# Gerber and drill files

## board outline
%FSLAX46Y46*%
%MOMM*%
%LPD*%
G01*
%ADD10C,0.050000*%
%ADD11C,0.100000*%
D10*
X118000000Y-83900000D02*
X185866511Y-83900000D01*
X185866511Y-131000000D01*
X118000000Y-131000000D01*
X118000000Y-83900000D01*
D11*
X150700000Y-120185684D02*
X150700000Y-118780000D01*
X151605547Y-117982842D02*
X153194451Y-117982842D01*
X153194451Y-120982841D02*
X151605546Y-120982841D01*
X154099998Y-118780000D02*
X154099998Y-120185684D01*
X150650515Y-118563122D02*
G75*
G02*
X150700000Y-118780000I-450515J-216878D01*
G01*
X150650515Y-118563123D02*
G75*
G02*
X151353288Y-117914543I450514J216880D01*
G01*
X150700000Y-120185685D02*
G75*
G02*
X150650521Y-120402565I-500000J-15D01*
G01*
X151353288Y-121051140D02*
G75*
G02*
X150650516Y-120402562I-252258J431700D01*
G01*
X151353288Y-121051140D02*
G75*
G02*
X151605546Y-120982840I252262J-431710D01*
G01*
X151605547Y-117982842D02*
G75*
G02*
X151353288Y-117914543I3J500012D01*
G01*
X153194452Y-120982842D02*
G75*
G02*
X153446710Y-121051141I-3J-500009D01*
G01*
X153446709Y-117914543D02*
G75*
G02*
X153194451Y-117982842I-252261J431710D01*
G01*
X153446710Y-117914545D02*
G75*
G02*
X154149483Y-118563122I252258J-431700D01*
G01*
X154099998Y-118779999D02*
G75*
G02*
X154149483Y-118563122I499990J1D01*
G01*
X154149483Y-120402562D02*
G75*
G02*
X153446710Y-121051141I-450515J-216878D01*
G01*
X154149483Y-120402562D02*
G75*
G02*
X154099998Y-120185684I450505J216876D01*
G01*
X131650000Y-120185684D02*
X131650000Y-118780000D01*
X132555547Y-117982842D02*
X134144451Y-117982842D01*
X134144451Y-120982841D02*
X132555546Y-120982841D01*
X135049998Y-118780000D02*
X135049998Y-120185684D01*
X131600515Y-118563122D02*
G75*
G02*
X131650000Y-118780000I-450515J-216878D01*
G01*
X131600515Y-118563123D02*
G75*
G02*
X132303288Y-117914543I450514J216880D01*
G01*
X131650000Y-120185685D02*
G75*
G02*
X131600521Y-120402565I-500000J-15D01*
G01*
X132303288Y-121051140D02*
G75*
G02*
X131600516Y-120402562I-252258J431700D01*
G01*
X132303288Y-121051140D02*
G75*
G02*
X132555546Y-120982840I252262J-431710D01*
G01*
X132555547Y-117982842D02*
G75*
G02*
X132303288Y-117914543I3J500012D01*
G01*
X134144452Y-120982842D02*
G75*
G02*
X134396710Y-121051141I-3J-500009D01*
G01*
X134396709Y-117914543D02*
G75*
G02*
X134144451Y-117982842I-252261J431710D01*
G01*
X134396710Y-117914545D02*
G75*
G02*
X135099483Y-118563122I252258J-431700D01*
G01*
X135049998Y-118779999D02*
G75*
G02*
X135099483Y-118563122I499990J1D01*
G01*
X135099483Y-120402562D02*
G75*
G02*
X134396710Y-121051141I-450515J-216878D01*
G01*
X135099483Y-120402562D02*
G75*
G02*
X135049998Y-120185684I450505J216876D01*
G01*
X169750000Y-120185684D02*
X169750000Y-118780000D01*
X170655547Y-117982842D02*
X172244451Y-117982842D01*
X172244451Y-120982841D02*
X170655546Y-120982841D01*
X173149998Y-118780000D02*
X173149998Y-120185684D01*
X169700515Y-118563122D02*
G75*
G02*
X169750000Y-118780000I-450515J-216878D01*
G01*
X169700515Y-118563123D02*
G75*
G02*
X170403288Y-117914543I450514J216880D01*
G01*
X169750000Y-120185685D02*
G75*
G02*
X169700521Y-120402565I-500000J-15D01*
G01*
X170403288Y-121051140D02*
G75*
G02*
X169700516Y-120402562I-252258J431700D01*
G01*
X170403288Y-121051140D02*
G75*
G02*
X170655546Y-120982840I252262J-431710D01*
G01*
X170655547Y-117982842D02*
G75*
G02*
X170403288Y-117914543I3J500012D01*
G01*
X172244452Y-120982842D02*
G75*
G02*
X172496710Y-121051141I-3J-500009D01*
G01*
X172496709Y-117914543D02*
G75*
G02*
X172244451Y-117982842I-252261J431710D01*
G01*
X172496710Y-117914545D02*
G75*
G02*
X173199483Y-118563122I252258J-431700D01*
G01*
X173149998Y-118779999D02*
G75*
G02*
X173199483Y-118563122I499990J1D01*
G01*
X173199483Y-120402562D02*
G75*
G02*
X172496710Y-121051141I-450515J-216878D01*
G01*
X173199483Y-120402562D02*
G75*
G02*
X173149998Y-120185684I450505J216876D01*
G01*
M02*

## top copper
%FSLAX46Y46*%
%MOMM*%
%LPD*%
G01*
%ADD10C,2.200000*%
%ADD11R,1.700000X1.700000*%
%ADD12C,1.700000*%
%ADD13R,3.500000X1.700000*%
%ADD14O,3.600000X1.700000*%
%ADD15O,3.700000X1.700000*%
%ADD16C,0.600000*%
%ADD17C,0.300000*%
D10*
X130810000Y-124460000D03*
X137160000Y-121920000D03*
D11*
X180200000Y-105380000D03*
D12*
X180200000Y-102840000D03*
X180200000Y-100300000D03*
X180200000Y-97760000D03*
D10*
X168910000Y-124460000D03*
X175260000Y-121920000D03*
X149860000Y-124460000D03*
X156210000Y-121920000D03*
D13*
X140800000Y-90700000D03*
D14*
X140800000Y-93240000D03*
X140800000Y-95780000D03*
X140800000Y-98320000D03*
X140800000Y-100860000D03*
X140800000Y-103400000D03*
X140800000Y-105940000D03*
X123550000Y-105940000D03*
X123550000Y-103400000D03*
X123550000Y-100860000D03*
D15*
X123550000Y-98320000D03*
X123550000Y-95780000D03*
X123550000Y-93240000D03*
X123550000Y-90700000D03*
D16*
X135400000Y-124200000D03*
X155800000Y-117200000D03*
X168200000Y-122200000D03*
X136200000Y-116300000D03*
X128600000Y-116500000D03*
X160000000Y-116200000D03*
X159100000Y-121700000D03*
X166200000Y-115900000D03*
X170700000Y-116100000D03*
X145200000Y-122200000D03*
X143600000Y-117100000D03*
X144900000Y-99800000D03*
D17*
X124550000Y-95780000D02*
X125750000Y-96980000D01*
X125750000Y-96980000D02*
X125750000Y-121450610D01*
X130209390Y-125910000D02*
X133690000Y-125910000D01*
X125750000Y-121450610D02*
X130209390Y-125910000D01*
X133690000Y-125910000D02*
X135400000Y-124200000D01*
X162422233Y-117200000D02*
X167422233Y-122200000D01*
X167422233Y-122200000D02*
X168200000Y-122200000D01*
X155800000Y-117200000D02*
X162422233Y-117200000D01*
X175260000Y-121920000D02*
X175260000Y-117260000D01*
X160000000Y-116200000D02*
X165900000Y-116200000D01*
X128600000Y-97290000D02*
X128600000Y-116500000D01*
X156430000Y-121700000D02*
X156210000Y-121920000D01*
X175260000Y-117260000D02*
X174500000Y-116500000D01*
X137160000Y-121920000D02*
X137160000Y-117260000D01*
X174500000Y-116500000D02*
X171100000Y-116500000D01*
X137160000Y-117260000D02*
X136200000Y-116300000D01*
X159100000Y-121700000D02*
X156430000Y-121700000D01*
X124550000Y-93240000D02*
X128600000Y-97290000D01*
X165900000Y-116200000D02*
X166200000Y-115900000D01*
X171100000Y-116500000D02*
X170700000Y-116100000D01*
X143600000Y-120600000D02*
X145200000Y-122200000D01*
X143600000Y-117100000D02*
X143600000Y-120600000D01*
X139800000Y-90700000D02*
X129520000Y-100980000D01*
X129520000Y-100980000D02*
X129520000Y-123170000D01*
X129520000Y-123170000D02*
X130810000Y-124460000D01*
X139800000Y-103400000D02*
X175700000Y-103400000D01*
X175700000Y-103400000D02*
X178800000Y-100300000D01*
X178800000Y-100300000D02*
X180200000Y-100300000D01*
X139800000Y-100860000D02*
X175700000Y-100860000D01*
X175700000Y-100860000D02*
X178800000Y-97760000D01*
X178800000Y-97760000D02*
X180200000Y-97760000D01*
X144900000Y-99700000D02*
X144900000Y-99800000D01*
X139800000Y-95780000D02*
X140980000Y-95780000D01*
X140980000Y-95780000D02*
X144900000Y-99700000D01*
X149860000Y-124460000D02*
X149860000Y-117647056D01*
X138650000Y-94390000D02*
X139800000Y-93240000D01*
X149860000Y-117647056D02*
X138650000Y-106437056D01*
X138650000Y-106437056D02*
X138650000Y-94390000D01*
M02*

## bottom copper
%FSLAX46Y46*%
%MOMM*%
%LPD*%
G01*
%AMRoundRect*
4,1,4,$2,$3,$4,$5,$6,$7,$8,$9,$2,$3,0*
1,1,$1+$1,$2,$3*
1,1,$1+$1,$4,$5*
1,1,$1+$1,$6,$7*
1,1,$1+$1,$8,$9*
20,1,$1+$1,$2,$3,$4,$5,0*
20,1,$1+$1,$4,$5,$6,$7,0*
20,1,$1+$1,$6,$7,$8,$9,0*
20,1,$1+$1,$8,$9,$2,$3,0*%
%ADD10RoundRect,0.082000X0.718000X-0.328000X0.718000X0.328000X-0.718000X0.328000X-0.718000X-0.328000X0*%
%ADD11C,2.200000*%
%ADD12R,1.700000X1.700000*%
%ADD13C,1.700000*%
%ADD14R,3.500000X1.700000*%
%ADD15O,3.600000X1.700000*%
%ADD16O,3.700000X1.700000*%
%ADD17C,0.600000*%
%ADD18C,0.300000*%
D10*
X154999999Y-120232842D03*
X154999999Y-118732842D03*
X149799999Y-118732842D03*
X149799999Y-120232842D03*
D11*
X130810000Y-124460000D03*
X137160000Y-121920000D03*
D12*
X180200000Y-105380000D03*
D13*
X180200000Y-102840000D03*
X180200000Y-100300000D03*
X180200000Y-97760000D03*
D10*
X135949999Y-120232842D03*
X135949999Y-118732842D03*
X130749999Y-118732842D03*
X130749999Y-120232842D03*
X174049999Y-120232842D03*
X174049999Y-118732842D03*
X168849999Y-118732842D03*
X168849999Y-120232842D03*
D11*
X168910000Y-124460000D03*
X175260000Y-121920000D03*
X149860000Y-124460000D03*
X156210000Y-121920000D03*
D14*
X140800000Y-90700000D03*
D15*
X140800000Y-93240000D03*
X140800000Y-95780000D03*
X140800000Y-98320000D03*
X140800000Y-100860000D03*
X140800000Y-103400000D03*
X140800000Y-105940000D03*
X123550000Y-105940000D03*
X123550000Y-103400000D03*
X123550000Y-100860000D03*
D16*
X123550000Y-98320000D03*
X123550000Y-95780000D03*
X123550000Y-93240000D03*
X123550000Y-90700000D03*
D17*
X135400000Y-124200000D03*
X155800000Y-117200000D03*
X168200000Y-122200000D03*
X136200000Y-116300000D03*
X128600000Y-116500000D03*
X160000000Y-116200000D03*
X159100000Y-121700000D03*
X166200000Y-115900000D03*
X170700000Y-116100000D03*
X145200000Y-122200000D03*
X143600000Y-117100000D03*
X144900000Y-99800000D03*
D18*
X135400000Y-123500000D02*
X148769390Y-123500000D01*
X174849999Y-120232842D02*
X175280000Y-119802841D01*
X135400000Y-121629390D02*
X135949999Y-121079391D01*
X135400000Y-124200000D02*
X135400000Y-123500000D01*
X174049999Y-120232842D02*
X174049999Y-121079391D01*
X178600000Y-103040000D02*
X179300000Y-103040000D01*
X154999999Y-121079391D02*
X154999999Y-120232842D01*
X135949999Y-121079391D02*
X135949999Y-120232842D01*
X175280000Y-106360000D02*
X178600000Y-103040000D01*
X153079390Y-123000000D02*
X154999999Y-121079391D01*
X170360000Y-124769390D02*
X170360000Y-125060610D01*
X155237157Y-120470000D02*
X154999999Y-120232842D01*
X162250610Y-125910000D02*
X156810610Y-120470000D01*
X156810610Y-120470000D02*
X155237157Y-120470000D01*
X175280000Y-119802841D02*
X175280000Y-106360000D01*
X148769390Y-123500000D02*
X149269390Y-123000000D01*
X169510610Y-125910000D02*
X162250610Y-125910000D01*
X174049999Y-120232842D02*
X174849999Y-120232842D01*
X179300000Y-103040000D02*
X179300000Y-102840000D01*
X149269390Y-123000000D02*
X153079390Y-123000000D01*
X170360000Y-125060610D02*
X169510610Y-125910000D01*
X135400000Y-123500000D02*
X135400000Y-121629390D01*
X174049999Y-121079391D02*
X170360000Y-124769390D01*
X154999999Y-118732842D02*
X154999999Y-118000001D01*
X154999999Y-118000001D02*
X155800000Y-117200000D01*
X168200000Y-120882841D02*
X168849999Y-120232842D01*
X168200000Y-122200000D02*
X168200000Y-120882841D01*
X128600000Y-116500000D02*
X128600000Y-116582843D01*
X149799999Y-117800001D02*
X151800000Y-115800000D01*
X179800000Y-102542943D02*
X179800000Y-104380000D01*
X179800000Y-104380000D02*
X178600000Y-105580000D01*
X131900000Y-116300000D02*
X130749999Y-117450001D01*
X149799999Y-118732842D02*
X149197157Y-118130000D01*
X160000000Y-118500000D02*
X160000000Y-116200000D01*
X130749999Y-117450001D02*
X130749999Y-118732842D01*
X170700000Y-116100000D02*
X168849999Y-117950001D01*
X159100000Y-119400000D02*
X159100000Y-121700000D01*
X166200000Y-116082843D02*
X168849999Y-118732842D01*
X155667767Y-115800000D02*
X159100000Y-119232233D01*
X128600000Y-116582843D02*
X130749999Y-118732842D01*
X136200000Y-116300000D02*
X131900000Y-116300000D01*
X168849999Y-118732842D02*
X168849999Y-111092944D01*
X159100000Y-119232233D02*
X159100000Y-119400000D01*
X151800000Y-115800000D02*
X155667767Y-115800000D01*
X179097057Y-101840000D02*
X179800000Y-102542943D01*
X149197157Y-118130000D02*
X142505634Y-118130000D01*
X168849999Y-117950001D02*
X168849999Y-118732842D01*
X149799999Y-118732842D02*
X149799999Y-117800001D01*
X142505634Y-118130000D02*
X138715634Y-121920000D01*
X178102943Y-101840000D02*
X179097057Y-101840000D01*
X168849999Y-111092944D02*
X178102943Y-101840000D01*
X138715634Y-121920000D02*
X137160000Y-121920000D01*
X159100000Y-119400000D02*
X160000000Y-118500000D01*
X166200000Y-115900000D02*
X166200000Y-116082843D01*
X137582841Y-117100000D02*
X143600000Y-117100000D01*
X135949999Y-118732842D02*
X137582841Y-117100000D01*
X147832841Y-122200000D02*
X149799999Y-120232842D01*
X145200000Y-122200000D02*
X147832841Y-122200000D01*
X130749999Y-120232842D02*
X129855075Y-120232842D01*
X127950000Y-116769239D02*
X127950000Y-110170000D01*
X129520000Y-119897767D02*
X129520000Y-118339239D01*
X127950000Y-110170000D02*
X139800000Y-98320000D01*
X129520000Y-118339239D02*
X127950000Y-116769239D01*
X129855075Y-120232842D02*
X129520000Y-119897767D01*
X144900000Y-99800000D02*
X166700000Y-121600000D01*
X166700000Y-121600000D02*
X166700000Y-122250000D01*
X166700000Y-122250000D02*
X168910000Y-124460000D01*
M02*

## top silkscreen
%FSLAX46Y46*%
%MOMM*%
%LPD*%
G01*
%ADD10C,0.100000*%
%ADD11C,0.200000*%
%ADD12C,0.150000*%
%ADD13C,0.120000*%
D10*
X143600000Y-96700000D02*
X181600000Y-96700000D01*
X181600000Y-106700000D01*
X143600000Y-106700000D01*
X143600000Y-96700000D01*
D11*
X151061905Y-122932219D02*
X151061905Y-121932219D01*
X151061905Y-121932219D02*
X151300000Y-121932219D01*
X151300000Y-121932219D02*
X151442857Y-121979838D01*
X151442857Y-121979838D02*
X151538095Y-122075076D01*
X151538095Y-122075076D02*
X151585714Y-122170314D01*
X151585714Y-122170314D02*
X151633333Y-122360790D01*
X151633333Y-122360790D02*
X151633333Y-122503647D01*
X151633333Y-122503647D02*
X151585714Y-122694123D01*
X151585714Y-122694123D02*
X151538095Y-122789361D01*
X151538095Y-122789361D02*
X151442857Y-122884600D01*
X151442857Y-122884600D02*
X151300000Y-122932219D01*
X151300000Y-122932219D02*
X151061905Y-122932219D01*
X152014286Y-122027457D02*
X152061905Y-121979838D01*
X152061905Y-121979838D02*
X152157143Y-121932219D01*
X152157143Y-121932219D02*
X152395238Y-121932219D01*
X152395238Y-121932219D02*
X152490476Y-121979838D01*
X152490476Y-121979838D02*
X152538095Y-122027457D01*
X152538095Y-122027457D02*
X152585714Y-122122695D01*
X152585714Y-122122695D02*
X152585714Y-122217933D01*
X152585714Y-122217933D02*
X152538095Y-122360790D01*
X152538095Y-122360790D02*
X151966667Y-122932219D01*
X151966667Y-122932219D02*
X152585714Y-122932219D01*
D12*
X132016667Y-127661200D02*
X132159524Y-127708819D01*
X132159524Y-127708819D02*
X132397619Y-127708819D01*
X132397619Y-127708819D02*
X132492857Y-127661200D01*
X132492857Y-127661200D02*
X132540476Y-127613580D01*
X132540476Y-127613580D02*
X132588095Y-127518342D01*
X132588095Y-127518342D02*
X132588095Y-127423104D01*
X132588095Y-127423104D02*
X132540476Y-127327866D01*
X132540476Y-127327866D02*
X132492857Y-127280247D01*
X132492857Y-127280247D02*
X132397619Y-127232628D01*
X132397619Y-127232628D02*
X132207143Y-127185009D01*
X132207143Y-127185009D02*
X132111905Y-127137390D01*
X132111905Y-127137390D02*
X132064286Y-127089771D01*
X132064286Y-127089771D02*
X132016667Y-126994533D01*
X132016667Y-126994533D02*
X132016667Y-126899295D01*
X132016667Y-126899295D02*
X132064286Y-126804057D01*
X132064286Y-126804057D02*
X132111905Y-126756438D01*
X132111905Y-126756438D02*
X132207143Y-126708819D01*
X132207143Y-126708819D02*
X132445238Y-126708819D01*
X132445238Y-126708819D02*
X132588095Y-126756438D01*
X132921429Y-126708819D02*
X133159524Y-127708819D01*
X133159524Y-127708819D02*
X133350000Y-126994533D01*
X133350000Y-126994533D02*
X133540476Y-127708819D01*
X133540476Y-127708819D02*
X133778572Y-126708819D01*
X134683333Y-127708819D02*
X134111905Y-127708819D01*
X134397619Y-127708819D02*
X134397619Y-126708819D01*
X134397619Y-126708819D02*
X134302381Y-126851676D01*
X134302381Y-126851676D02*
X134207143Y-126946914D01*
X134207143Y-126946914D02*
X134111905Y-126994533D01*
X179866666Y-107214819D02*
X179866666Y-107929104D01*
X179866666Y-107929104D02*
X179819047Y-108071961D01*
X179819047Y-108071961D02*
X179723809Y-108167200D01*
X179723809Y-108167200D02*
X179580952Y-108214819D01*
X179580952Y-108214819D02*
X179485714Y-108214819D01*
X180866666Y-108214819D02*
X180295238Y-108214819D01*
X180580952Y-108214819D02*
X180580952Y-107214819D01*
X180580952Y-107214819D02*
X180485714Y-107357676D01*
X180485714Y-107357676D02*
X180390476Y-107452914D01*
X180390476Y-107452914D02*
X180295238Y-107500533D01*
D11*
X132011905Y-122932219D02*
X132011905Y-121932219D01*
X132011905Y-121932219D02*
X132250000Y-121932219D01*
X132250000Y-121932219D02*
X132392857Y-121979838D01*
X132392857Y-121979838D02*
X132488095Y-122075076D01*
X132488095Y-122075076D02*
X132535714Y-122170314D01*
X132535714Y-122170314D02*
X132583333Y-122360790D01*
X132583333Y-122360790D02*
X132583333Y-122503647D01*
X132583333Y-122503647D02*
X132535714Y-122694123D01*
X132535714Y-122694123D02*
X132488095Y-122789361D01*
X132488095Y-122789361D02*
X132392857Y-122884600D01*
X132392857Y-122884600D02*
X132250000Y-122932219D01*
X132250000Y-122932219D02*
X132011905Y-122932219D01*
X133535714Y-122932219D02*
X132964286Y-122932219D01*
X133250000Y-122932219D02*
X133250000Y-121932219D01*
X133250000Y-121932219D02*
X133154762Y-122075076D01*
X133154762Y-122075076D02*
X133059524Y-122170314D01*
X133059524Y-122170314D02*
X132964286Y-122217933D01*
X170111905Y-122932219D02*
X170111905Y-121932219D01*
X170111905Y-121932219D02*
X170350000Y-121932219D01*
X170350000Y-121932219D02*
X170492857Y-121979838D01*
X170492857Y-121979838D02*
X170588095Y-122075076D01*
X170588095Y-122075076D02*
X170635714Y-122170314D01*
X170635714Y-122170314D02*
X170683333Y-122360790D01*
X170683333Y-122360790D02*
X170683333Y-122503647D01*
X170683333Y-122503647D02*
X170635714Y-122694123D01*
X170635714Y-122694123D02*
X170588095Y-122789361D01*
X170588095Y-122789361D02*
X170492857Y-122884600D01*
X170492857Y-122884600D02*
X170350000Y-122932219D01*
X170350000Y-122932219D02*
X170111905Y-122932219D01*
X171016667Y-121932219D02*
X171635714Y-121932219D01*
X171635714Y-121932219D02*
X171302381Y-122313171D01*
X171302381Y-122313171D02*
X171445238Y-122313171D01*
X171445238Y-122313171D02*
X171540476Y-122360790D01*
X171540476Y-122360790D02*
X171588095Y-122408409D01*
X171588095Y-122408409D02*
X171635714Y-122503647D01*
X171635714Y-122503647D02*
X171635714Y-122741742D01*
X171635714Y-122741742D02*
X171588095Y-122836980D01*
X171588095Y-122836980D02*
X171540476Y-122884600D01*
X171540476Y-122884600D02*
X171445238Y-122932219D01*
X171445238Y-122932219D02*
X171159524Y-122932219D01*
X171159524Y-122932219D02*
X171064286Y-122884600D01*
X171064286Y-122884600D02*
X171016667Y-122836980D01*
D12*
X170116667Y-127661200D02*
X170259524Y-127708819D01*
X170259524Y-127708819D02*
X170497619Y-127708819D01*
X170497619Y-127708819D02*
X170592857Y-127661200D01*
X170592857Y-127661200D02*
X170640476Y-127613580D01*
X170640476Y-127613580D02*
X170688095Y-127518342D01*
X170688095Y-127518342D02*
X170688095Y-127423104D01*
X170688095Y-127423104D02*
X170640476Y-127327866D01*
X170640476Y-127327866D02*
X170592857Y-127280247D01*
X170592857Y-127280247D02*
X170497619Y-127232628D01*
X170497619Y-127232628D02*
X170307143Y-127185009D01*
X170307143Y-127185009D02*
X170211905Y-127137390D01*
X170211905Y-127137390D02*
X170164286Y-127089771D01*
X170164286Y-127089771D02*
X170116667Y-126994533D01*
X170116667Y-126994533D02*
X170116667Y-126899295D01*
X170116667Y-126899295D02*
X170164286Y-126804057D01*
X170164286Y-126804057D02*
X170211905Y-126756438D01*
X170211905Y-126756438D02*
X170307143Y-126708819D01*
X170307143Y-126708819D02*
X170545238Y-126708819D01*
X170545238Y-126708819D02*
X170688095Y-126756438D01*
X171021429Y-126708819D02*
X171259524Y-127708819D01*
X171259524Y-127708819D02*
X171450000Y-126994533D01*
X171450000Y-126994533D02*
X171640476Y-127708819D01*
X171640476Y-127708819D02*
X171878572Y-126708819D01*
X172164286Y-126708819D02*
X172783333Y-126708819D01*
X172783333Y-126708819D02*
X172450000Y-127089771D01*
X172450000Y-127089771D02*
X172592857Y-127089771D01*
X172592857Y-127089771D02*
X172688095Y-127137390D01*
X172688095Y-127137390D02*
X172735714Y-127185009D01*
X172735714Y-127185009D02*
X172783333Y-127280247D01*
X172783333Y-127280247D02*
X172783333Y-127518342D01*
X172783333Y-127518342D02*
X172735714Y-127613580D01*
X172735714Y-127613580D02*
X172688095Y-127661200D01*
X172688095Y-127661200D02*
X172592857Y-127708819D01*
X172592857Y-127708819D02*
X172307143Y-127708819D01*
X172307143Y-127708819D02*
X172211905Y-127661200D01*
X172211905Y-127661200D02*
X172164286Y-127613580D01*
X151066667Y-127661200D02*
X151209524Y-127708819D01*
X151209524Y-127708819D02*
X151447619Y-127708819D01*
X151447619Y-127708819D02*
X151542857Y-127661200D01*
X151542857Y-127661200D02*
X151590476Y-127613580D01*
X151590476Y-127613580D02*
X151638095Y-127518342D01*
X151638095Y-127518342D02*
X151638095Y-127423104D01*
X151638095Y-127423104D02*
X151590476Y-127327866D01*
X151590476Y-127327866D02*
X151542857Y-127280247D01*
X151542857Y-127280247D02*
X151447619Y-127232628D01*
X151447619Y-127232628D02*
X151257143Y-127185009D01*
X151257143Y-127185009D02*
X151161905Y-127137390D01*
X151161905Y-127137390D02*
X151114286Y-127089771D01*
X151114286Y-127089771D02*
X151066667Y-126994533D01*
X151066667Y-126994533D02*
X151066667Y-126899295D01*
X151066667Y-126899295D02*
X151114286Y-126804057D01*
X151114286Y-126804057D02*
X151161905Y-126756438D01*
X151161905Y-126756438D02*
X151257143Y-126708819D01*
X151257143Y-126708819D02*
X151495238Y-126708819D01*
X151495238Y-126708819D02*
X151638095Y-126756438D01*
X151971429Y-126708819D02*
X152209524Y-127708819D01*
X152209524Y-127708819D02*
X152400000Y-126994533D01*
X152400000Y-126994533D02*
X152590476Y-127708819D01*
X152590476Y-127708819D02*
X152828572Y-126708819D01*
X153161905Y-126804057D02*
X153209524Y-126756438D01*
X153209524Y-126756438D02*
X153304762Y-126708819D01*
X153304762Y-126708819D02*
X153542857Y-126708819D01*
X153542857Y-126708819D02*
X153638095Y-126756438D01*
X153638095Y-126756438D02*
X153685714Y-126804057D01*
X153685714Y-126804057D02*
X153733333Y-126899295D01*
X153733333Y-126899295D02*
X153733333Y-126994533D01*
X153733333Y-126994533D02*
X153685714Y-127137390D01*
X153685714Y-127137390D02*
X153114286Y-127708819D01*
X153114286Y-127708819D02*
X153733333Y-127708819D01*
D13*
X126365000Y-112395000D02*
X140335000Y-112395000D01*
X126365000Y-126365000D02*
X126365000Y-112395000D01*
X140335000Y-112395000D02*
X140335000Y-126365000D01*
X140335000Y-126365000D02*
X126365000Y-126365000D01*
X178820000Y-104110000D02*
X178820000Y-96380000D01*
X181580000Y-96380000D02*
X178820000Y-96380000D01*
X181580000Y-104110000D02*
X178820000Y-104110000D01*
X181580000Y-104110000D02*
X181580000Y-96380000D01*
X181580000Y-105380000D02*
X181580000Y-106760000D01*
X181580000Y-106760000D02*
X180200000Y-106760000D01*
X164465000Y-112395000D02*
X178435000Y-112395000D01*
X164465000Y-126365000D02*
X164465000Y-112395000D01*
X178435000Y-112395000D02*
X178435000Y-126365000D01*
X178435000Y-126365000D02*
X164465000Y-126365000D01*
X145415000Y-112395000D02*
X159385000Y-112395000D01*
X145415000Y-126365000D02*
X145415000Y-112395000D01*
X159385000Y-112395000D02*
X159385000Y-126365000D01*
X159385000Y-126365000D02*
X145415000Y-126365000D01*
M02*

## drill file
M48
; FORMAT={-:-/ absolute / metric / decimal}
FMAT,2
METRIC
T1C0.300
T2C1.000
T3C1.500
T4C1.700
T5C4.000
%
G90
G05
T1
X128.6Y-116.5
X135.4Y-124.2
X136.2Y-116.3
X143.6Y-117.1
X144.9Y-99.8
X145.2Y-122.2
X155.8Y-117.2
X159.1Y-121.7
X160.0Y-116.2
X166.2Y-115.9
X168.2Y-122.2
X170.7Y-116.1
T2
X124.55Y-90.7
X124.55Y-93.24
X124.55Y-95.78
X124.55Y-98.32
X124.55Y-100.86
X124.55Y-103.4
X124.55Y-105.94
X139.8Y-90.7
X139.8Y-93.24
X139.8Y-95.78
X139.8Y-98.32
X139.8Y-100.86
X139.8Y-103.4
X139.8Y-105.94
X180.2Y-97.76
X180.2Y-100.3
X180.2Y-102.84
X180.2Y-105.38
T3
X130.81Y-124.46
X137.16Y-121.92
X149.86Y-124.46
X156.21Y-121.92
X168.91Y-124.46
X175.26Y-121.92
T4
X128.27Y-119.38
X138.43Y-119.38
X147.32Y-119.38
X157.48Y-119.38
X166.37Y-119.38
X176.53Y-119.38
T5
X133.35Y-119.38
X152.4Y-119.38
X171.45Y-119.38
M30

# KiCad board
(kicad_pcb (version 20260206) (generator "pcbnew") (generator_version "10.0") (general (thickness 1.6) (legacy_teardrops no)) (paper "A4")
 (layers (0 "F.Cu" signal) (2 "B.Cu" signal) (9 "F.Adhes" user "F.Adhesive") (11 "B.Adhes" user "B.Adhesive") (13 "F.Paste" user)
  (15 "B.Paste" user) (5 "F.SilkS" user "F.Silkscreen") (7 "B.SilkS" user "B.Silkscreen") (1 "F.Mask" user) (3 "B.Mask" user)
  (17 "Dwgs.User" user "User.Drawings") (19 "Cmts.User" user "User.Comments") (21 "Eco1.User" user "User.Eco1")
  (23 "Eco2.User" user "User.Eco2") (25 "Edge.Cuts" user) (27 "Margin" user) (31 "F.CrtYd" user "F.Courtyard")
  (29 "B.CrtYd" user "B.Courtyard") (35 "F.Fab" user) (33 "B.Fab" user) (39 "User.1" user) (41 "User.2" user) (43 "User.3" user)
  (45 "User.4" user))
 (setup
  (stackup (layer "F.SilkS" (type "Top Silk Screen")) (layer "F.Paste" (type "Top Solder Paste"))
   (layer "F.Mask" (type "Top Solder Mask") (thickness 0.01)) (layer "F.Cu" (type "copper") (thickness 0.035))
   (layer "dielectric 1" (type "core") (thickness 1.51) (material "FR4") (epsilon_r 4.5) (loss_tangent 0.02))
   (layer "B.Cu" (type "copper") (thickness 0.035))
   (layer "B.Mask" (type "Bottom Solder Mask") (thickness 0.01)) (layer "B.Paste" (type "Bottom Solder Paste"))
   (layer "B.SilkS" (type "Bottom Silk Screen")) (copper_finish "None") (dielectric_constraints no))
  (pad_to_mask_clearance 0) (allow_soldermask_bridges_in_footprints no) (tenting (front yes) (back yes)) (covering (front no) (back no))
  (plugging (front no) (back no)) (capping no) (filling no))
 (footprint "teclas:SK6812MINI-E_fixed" (layer "F.Cu") (at 152.4 119.38 180)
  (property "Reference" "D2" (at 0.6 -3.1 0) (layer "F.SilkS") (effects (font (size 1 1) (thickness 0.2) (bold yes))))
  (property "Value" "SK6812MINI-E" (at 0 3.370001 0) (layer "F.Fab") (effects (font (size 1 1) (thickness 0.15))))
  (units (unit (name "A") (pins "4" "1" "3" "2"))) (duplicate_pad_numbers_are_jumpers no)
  (fp_line (start 1.7 -0.805684) (end 1.7 0.6) (stroke (width 0.1) (type solid)) (layer "Edge.Cuts"))
  (fp_line (start 0.794453 1.397158) (end -0.794451 1.397158) (stroke (width 0.1) (type solid)) (layer "Edge.Cuts"))
  (fp_line (start -0.794451 -1.602841) (end 0.794454 -1.602841) (stroke (width 0.1) (type solid)) (layer "Edge.Cuts"))
  (fp_line (start -1.699998 0.6) (end -1.699998 -0.805684) (stroke (width 0.1) (type solid)) (layer "Edge.Cuts"))
  (fp_arc (start 1.749485 0.816878) (mid 1.712528 0.711226) (end 1.7 0.6) (stroke (width 0.1) (type solid)) (layer "Edge.Cuts"))
  (fp_arc (start 1.749485 0.816877) (mid 1.638073 1.401193) (end 1.046712 1.465457) (stroke (width 0.1) (type solid)) (layer "Edge.Cuts"))
  (fp_arc (start 1.7 -0.805685) (mid 1.712528 -0.91691) (end 1.749485 -1.022562) (stroke (width 0.1) (type solid)) (layer "Edge.Cuts"))
  (fp_arc (start 1.046712 -1.67114) (mid 1.638072 -1.606876) (end 1.749485 -1.022562) (stroke (width 0.1) (type solid)) (layer "Edge.Cuts"))
  (fp_arc (start 1.046712 -1.67114) (mid 0.925124 -1.620218) (end 0.794454 -1.602841) (stroke (width 0.1) (type solid)) (layer "Edge.Cuts"))
  (fp_arc (start 0.794453 1.397158) (mid 0.925124 1.414535) (end 1.046712 1.465457) (stroke (width 0.1) (type solid)) (layer "Edge.Cuts"))
  (fp_arc (start -0.794452 -1.602842) (mid -0.925122 -1.620219) (end -1.04671 -1.671141) (stroke (width 0.1) (type solid))
   (layer "Edge.Cuts"))
  (fp_arc (start -1.046709 1.465457) (mid -0.925121 1.414535) (end -0.794451 1.397158) (stroke (width 0.1) (type solid)) (layer "Edge.Cuts"))
  (fp_arc (start -1.04671 1.465455) (mid -1.638069 1.401192) (end -1.749483 0.816878) (stroke (width 0.1) (type solid)) (layer "Edge.Cuts"))
  (fp_arc (start -1.699998 0.600001) (mid -1.712526 0.711226) (end -1.749483 0.816878) (stroke (width 0.1) (type solid)) (layer "Edge.Cuts"))
  (fp_arc (start -1.749483 -1.022562) (mid -1.63807 -1.606877) (end -1.04671 -1.671141) (stroke (width 0.1) (type solid))
   (layer "Edge.Cuts"))
  (fp_arc (start -1.749483 -1.022562) (mid -1.712526 -0.91691) (end -1.699998 -0.805684) (stroke (width 0.1) (type solid))
   (layer "Edge.Cuts"))
  (pad "1" smd roundrect (at -2.599999 -0.852842 90) (size 0.82 1.6) (layers "B.Cu" "B.Mask" "B.Paste") (roundrect_rratio 0.1) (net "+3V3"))
  (pad "2" smd roundrect (at -2.599999 0.647158 90) (size 0.82 1.6) (layers "B.Cu" "B.Mask" "B.Paste") (roundrect_rratio 0.1)
   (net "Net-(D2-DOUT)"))
  (pad "3" smd roundrect (at 2.600001 0.647158 90) (size 0.82 1.6) (layers "B.Cu" "B.Mask" "B.Paste") (roundrect_rratio 0.1) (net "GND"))
  (pad "4" smd roundrect (at 2.600001 -0.852842 90) (size 0.82 1.6) (layers "B.Cu" "B.Mask" "B.Paste") (roundrect_rratio 0.1)
   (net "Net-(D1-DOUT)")))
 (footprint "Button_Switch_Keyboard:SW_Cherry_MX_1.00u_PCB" (layer "F.Cu") (at 130.81 124.46 180)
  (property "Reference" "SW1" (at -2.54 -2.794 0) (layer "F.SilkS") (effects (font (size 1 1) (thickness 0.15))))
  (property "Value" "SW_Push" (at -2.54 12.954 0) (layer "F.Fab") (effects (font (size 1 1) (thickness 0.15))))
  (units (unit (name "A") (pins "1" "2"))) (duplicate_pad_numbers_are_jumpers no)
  (fp_line (start 4.445 12.065) (end -9.525 12.065) (stroke (width 0.12) (type solid)) (layer "F.SilkS"))
  (fp_line (start 4.445 -1.905) (end 4.445 12.065) (stroke (width 0.12) (type solid)) (layer "F.SilkS"))
  (fp_line (start -9.525 12.065) (end -9.525 -1.905) (stroke (width 0.12) (type solid)) (layer "F.SilkS"))
  (fp_line (start -9.525 -1.905) (end 4.445 -1.905) (stroke (width 0.12) (type solid)) (layer "F.SilkS"))
  (pad "" np_thru_hole circle (at -7.62 5.08 180) (size 1.7 1.7) (drill 1.7) (layers "*.Cu" "*.Mask"))
  (pad "" np_thru_hole circle (at -2.54 5.08 180) (size 4 4) (drill 4) (layers "*.Cu" "*.Mask"))
  (pad "" np_thru_hole circle (at 2.54 5.08 180) (size 1.7 1.7) (drill 1.7) (layers "*.Cu" "*.Mask"))
  (pad "1" thru_hole circle (at 0 0 180) (size 2.2 2.2) (drill 1.5) (layers "*.Cu" "*.Mask") (remove_unused_layers no)
   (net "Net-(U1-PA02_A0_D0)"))
  (pad "2" thru_hole circle (at -6.35 2.54 180) (size 2.2 2.2) (drill 1.5) (layers "*.Cu" "*.Mask") (remove_unused_layers no) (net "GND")))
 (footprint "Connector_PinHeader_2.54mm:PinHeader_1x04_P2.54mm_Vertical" (layer "F.Cu") (at 180.2 105.38 180)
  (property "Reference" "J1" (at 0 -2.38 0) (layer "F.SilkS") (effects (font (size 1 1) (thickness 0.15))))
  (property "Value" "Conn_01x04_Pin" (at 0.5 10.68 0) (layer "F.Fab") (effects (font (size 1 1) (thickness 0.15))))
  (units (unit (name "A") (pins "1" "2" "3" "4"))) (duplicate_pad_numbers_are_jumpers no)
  (fp_line (start 1.38 1.27) (end 1.38 9) (stroke (width 0.12) (type solid)) (layer "F.SilkS"))
  (fp_line (start -1.38 9) (end 1.38 9) (stroke (width 0.12) (type solid)) (layer "F.SilkS"))
  (fp_line (start -1.38 1.27) (end 1.38 1.27) (stroke (width 0.12) (type solid)) (layer "F.SilkS"))
  (fp_line (start -1.38 1.27) (end -1.38 9) (stroke (width 0.12) (type solid)) (layer "F.SilkS"))
  (fp_line (start -1.38 0) (end -1.38 -1.38) (stroke (width 0.12) (type solid)) (layer "F.SilkS"))
  (fp_line (start -1.38 -1.38) (end 0 -1.38) (stroke (width 0.12) (type solid)) (layer "F.SilkS"))
  (pad "1" thru_hole rect (at 0 0 180) (size 1.7 1.7) (drill 1) (layers "*.Cu" "*.Mask") (remove_unused_layers no) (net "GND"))
  (pad "2" thru_hole circle (at 0 2.54 180) (size 1.7 1.7) (drill 1) (layers "*.Cu" "*.Mask") (remove_unused_layers no) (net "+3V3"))
  (pad "3" thru_hole circle (at 0 5.08 180) (size 1.7 1.7) (drill 1) (layers "*.Cu" "*.Mask") (remove_unused_layers no)
   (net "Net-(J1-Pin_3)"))
  (pad "4" thru_hole circle (at 0 7.62 180) (size 1.7 1.7) (drill 1) (layers "*.Cu" "*.Mask") (remove_unused_layers no)
   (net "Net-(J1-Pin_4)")))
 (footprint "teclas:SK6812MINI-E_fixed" (layer "F.Cu") (at 133.35 119.38 180)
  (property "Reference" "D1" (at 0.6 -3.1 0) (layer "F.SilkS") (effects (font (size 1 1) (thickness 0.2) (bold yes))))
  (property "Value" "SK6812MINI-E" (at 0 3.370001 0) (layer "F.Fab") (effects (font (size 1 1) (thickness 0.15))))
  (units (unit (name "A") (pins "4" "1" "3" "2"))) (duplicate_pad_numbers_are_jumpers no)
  (fp_line (start 1.7 -0.805684) (end 1.7 0.6) (stroke (width 0.1) (type solid)) (layer "Edge.Cuts"))
  (fp_line (start 0.794453 1.397158) (end -0.794451 1.397158) (stroke (width 0.1) (type solid)) (layer "Edge.Cuts"))
  (fp_line (start -0.794451 -1.602841) (end 0.794454 -1.602841) (stroke (width 0.1) (type solid)) (layer "Edge.Cuts"))
  (fp_line (start -1.699998 0.6) (end -1.699998 -0.805684) (stroke (width 0.1) (type solid)) (layer "Edge.Cuts"))
  (fp_arc (start 1.749485 0.816878) (mid 1.712528 0.711226) (end 1.7 0.6) (stroke (width 0.1) (type solid)) (layer "Edge.Cuts"))
  (fp_arc (start 1.749485 0.816877) (mid 1.638073 1.401193) (end 1.046712 1.465457) (stroke (width 0.1) (type solid)) (layer "Edge.Cuts"))
  (fp_arc (start 1.7 -0.805685) (mid 1.712528 -0.91691) (end 1.749485 -1.022562) (stroke (width 0.1) (type solid)) (layer "Edge.Cuts"))
  (fp_arc (start 1.046712 -1.67114) (mid 1.638072 -1.606876) (end 1.749485 -1.022562) (stroke (width 0.1) (type solid)) (layer "Edge.Cuts"))
  (fp_arc (start 1.046712 -1.67114) (mid 0.925124 -1.620218) (end 0.794454 -1.602841) (stroke (width 0.1) (type solid)) (layer "Edge.Cuts"))
  (fp_arc (start 0.794453 1.397158) (mid 0.925124 1.414535) (end 1.046712 1.465457) (stroke (width 0.1) (type solid)) (layer "Edge.Cuts"))
  (fp_arc (start -0.794452 -1.602842) (mid -0.925122 -1.620219) (end -1.04671 -1.671141) (stroke (width 0.1) (type solid))
   (layer "Edge.Cuts"))
  (fp_arc (start -1.046709 1.465457) (mid -0.925121 1.414535) (end -0.794451 1.397158) (stroke (width 0.1) (type solid)) (layer "Edge.Cuts"))
  (fp_arc (start -1.04671 1.465455) (mid -1.638069 1.401192) (end -1.749483 0.816878) (stroke (width 0.1) (type solid)) (layer "Edge.Cuts"))
  (fp_arc (start -1.699998 0.600001) (mid -1.712526 0.711226) (end -1.749483 0.816878) (stroke (width 0.1) (type solid)) (layer "Edge.Cuts"))
  (fp_arc (start -1.749483 -1.022562) (mid -1.63807 -1.606877) (end -1.04671 -1.671141) (stroke (width 0.1) (type solid))
   (layer "Edge.Cuts"))
  (fp_arc (start -1.749483 -1.022562) (mid -1.712526 -0.91691) (end -1.699998 -0.805684) (stroke (width 0.1) (type solid))
   (layer "Edge.Cuts"))
  (pad "1" smd roundrect (at -2.599999 -0.852842 90) (size 0.82 1.6) (layers "B.Cu" "B.Mask" "B.Paste") (roundrect_rratio 0.1) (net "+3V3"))
  (pad "2" smd roundrect (at -2.599999 0.647158 90) (size 0.82 1.6) (layers "B.Cu" "B.Mask" "B.Paste") (roundrect_rratio 0.1)
   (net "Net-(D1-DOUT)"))
  (pad "3" smd roundrect (at 2.600001 0.647158 90) (size 0.82 1.6) (layers "B.Cu" "B.Mask" "B.Paste") (roundrect_rratio 0.1) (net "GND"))
  (pad "4" smd roundrect (at 2.600001 -0.852842 90) (size 0.82 1.6) (layers "B.Cu" "B.Mask" "B.Paste") (roundrect_rratio 0.1)
   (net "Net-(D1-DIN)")))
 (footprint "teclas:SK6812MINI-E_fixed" (layer "F.Cu") (at 171.45 119.38 180)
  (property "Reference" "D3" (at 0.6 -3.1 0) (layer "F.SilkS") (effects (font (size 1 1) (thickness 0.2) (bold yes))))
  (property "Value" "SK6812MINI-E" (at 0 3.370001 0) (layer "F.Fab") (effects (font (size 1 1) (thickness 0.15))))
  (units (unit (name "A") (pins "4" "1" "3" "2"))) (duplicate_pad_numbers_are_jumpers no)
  (fp_line (start 1.7 -0.805684) (end 1.7 0.6) (stroke (width 0.1) (type solid)) (layer "Edge.Cuts"))
  (fp_line (start 0.794453 1.397158) (end -0.794451 1.397158) (stroke (width 0.1) (type solid)) (layer "Edge.Cuts"))
  (fp_line (start -0.794451 -1.602841) (end 0.794454 -1.602841) (stroke (width 0.1) (type solid)) (layer "Edge.Cuts"))
  (fp_line (start -1.699998 0.6) (end -1.699998 -0.805684) (stroke (width 0.1) (type solid)) (layer "Edge.Cuts"))
  (fp_arc (start 1.749485 0.816878) (mid 1.712528 0.711226) (end 1.7 0.6) (stroke (width 0.1) (type solid)) (layer "Edge.Cuts"))
  (fp_arc (start 1.749485 0.816877) (mid 1.638073 1.401193) (end 1.046712 1.465457) (stroke (width 0.1) (type solid)) (layer "Edge.Cuts"))
  (fp_arc (start 1.7 -0.805685) (mid 1.712528 -0.91691) (end 1.749485 -1.022562) (stroke (width 0.1) (type solid)) (layer "Edge.Cuts"))
  (fp_arc (start 1.046712 -1.67114) (mid 1.638072 -1.606876) (end 1.749485 -1.022562) (stroke (width 0.1) (type solid)) (layer "Edge.Cuts"))
  (fp_arc (start 1.046712 -1.67114) (mid 0.925124 -1.620218) (end 0.794454 -1.602841) (stroke (width 0.1) (type solid)) (layer "Edge.Cuts"))
  (fp_arc (start 0.794453 1.397158) (mid 0.925124 1.414535) (end 1.046712 1.465457) (stroke (width 0.1) (type solid)) (layer "Edge.Cuts"))
  (fp_arc (start -0.794452 -1.602842) (mid -0.925122 -1.620219) (end -1.04671 -1.671141) (stroke (width 0.1) (type solid))
   (layer "Edge.Cuts"))
  (fp_arc (start -1.046709 1.465457) (mid -0.925121 1.414535) (end -0.794451 1.397158) (stroke (width 0.1) (type solid)) (layer "Edge.Cuts"))
  (fp_arc (start -1.04671 1.465455) (mid -1.638069 1.401192) (end -1.749483 0.816878) (stroke (width 0.1) (type solid)) (layer "Edge.Cuts"))
  (fp_arc (start -1.699998 0.600001) (mid -1.712526 0.711226) (end -1.749483 0.816878) (stroke (width 0.1) (type solid)) (layer "Edge.Cuts"))
  (fp_arc (start -1.749483 -1.022562) (mid -1.63807 -1.606877) (end -1.04671 -1.671141) (stroke (width 0.1) (type solid))
   (layer "Edge.Cuts"))
  (fp_arc (start -1.749483 -1.022562) (mid -1.712526 -0.91691) (end -1.699998 -0.805684) (stroke (width 0.1) (type solid))
   (layer "Edge.Cuts"))
  (pad "1" smd roundrect (at -2.599999 -0.852842 90) (size 0.82 1.6) (layers "B.Cu" "B.Mask" "B.Paste") (roundrect_rratio 0.1) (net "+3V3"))
  (pad "2" smd roundrect (at -2.599999 0.647158 90) (size 0.82 1.6) (layers "B.Cu" "B.Mask" "B.Paste") (roundrect_rratio 0.1)
   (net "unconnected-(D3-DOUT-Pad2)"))
  (pad "3" smd roundrect (at 2.600001 0.647158 90) (size 0.82 1.6) (layers "B.Cu" "B.Mask" "B.Paste") (roundrect_rratio 0.1) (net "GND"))
  (pad "4" smd roundrect (at 2.600001 -0.852842 90) (size 0.82 1.6) (layers "B.Cu" "B.Mask" "B.Paste") (roundrect_rratio 0.1)
   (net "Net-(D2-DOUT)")))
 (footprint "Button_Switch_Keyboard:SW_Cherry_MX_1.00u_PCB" (layer "F.Cu") (at 168.91 124.46 180)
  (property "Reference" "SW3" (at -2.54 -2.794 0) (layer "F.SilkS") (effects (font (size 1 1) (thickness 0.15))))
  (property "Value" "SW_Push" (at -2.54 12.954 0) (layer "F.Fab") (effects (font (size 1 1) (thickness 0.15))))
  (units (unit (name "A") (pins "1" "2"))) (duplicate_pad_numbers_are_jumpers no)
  (fp_line (start 4.445 12.065) (end -9.525 12.065) (stroke (width 0.12) (type solid)) (layer "F.SilkS"))
  (fp_line (start 4.445 -1.905) (end 4.445 12.065) (stroke (width 0.12) (type solid)) (layer "F.SilkS"))
  (fp_line (start -9.525 12.065) (end -9.525 -1.905) (stroke (width 0.12) (type solid)) (layer "F.SilkS"))
  (fp_line (start -9.525 -1.905) (end 4.445 -1.905) (stroke (width 0.12) (type solid)) (layer "F.SilkS"))
  (pad "" np_thru_hole circle (at -7.62 5.08 180) (size 1.7 1.7) (drill 1.7) (layers "*.Cu" "*.Mask"))
  (pad "" np_thru_hole circle (at -2.54 5.08 180) (size 4 4) (drill 4) (layers "*.Cu" "*.Mask"))
  (pad "" np_thru_hole circle (at 2.54 5.08 180) (size 1.7 1.7) (drill 1.7) (layers "*.Cu" "*.Mask"))
  (pad "1" thru_hole circle (at 0 0 180) (size 2.2 2.2) (drill 1.5) (layers "*.Cu" "*.Mask") (remove_unused_layers no)
   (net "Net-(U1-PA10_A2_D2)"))
  (pad "2" thru_hole circle (at -6.35 2.54 180) (size 2.2 2.2) (drill 1.5) (layers "*.Cu" "*.Mask") (remove_unused_layers no) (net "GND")))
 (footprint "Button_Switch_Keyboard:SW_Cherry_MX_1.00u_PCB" (layer "F.Cu") (at 149.86 124.46 180)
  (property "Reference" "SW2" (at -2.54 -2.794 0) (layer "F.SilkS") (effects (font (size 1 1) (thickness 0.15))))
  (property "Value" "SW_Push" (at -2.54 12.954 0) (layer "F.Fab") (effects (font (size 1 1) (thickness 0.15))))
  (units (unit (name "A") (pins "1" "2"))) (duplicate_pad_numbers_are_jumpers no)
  (fp_line (start 4.445 12.065) (end -9.525 12.065) (stroke (width 0.12) (type solid)) (layer "F.SilkS"))
  (fp_line (start 4.445 -1.905) (end 4.445 12.065) (stroke (width 0.12) (type solid)) (layer "F.SilkS"))
  (fp_line (start -9.525 12.065) (end -9.525 -1.905) (stroke (width 0.12) (type solid)) (layer "F.SilkS"))
  (fp_line (start -9.525 -1.905) (end 4.445 -1.905) (stroke (width 0.12) (type solid)) (layer "F.SilkS"))
  (pad "" np_thru_hole circle (at -7.62 5.08 180) (size 1.7 1.7) (drill 1.7) (layers "*.Cu" "*.Mask"))
  (pad "" np_thru_hole circle (at -2.54 5.08 180) (size 4 4) (drill 4) (layers "*.Cu" "*.Mask"))
  (pad "" np_thru_hole circle (at 2.54 5.08 180) (size 1.7 1.7) (drill 1.7) (layers "*.Cu" "*.Mask"))
  (pad "1" thru_hole circle (at 0 0 180) (size 2.2 2.2) (drill 1.5) (layers "*.Cu" "*.Mask") (remove_unused_layers no)
   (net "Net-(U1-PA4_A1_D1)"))
  (pad "2" thru_hole circle (at -6.35 2.54 180) (size 2.2 2.2) (drill 1.5) (layers "*.Cu" "*.Mask") (remove_unused_layers no) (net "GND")))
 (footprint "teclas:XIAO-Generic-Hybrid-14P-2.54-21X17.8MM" (layer "B.Cu") (at 132.175 98.32 180)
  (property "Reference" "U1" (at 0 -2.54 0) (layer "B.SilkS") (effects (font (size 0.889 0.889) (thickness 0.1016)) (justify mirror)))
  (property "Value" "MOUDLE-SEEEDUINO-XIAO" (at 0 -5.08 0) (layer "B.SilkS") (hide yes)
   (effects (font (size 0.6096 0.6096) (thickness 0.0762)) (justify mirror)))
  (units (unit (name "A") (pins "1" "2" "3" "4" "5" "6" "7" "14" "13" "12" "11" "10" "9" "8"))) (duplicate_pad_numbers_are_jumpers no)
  (pad "1" thru_hole rect (at -7.625 7.62 180) (size 3.5 1.7) (drill 1 (offset -1 0)) (layers "*.Cu" "*.Mask") (remove_unused_layers no)
   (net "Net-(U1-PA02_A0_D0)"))
  (pad "2" thru_hole oval (at -7.625 5.08 180) (size 3.6 1.7) (drill 1 (offset -1 0)) (layers "*.Cu" "*.Mask") (remove_unused_layers no)
   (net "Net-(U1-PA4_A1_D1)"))
  (pad "3" thru_hole oval (at -7.625 2.54 180) (size 3.6 1.7) (drill 1 (offset -1 0)) (layers "*.Cu" "*.Mask") (remove_unused_layers no)
   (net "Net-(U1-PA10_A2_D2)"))
  (pad "4" thru_hole oval (at -7.625 0 180) (size 3.6 1.7) (drill 1 (offset -1 0)) (layers "*.Cu" "*.Mask") (remove_unused_layers no)
   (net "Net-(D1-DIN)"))
  (pad "5" thru_hole oval (at -7.625 -2.54 180) (size 3.6 1.7) (drill 1 (offset -1 0)) (layers "*.Cu" "*.Mask") (remove_unused_layers no)
   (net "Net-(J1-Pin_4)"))
  (pad "6" thru_hole oval (at -7.625 -5.08) (size 3.6 1.7) (drill 1 (offset 1 0)) (layers "*.Cu" "*.Mask") (remove_unused_layers no)
   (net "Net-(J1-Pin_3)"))
  (pad "7" thru_hole oval (at -7.625 -7.62 180) (size 3.6 1.7) (drill 1 (offset -1 0)) (layers "*.Cu" "*.Mask") (remove_unused_layers no)
   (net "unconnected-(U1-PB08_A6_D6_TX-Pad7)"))
  (pad "8" thru_hole oval (at 7.625 -7.62 180) (size 3.6 1.7) (drill 1 (offset 1 0)) (layers "*.Cu" "*.Mask") (remove_unused_layers no)
   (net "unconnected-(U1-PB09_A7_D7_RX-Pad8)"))
  (pad "9" thru_hole oval (at 7.625 -5.08 180) (size 3.6 1.7) (drill 1 (offset 1 0)) (layers "*.Cu" "*.Mask") (remove_unused_layers no)
   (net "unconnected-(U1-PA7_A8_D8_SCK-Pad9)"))
  (pad "10" thru_hole oval (at 7.625 -2.54 180) (size 3.6 1.7) (drill 1 (offset 1 0)) (layers "*.Cu" "*.Mask") (remove_unused_layers no)
   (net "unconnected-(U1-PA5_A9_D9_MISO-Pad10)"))
  (pad "11" thru_hole oval (at 7.625 0 180) (size 3.7 1.7) (drill 1 (offset 1 0)) (layers "*.Cu" "*.Mask") (remove_unused_layers no)
   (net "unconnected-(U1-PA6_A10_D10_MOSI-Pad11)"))
  (pad "12" thru_hole oval (at 7.625 2.54 180) (size 3.7 1.7) (drill 1 (offset 1 0)) (layers "*.Cu" "*.Mask") (remove_unused_layers no)
   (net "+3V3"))
  (pad "13" thru_hole oval (at 7.625 5.08 180) (size 3.7 1.7) (drill 1 (offset 1 0)) (layers "*.Cu" "*.Mask") (remove_unused_layers no)
   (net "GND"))
  (pad "14" thru_hole oval (at 7.625 7.62 180) (size 3.7 1.7) (drill 1 (offset 1 0)) (layers "*.Cu" "*.Mask") (remove_unused_layers no)
   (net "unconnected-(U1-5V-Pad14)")))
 (gr_rect (start 143.6 96.7) (end 181.6 106.7) (stroke (width 0.1) (type default)) (fill no) (layer "F.SilkS"))
 (gr_rect (start 118 83.9) (end 185.866511 131) (stroke (width 0.05) (type default)) (fill no) (layer "Edge.Cuts"))
 (segment (start 124.55 95.78) (end 125.75 96.98) (width 0.3) (layer "F.Cu") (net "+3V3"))
 (segment (start 125.75 96.98) (end 125.75 121.45061) (width 0.3) (layer "F.Cu") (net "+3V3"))
 (segment (start 130.20939 125.91) (end 133.69 125.91) (width 0.3) (layer "F.Cu") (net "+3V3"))
 (segment (start 125.75 121.45061) (end 130.20939 125.91) (width 0.3) (layer "F.Cu") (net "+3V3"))
 (segment (start 133.69 125.91) (end 135.4 124.2) (width 0.3) (layer "F.Cu") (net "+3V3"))
 (via (at 135.4 124.2) (size 0.6) (drill 0.3) (layers "F.Cu" "B.Cu") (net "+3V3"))
 (segment (start 135.4 123.5) (end 148.76939 123.5) (width 0.3) (layer "B.Cu") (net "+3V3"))
 (segment (start 174.849999 120.232842) (end 175.28 119.802841) (width 0.3) (layer "B.Cu") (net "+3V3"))
 (segment (start 135.4 121.62939) (end 135.949999 121.079391) (width 0.3) (layer "B.Cu") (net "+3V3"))
 (segment (start 135.4 124.2) (end 135.4 123.5) (width 0.3) (layer "B.Cu") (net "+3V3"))
 (segment (start 174.049999 120.232842) (end 174.049999 121.079391) (width 0.3) (layer "B.Cu") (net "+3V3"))
 (segment (start 178.6 103.04) (end 179.3 103.04) (width 0.3) (layer "B.Cu") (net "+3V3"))
 (segment (start 154.999999 121.079391) (end 154.999999 120.232842) (width 0.3) (layer "B.Cu") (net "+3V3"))
 (segment (start 135.949999 121.079391) (end 135.949999 120.232842) (width 0.3) (layer "B.Cu") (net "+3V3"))
 (segment (start 175.28 106.36) (end 178.6 103.04) (width 0.3) (layer "B.Cu") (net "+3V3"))
 (segment (start 153.07939 123) (end 154.999999 121.079391) (width 0.3) (layer "B.Cu") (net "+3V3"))
 (segment (start 170.36 124.76939) (end 170.36 125.06061) (width 0.3) (layer "B.Cu") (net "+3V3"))
 (segment (start 155.237157 120.47) (end 154.999999 120.232842) (width 0.3) (layer "B.Cu") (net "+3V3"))
 (segment (start 162.25061 125.91) (end 156.81061 120.47) (width 0.3) (layer "B.Cu") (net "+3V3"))
 (segment (start 156.81061 120.47) (end 155.237157 120.47) (width 0.3) (layer "B.Cu") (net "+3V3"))
 (segment (start 175.28 119.802841) (end 175.28 106.36) (width 0.3) (layer "B.Cu") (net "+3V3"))
 (segment (start 148.76939 123.5) (end 149.26939 123) (width 0.3) (layer "B.Cu") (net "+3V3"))
 (segment (start 169.51061 125.91) (end 162.25061 125.91) (width 0.3) (layer "B.Cu") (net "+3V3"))
 (segment (start 174.049999 120.232842) (end 174.849999 120.232842) (width 0.3) (layer "B.Cu") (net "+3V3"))
 (segment (start 179.3 103.04) (end 179.3 102.84) (width 0.3) (layer "B.Cu") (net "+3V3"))
 (segment (start 149.26939 123) (end 153.07939 123) (width 0.3) (layer "B.Cu") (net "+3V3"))
 (segment (start 170.36 125.06061) (end 169.51061 125.91) (width 0.3) (layer "B.Cu") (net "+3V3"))
 (segment (start 135.4 123.5) (end 135.4 121.62939) (width 0.3) (layer "B.Cu") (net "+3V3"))
 (segment (start 174.049999 121.079391) (end 170.36 124.76939) (width 0.3) (layer "B.Cu") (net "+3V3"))
 (segment (start 162.422233 117.2) (end 167.422233 122.2) (width 0.3) (layer "F.Cu") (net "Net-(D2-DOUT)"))
 (segment (start 167.422233 122.2) (end 168.2 122.2) (width 0.3) (layer "F.Cu") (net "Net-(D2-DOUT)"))
 (segment (start 155.8 117.2) (end 162.422233 117.2) (width 0.3) (layer "F.Cu") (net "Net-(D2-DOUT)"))
 (via (at 155.8 117.2) (size 0.6) (drill 0.3) (layers "F.Cu" "B.Cu") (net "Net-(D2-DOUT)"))
 (via (at 168.2 122.2) (size 0.6) (drill 0.3) (layers "F.Cu" "B.Cu") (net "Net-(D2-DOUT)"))
 (segment (start 154.999999 118.732842) (end 154.999999 118.000001) (width 0.3) (layer "B.Cu") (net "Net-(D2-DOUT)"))
 (segment (start 154.999999 118.000001) (end 155.8 117.2) (width 0.3) (layer "B.Cu") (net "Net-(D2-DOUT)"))
 (segment (start 168.2 120.882841) (end 168.849999 120.232842) (width 0.3) (layer "B.Cu") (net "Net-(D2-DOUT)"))
 (segment (start 168.2 122.2) (end 168.2 120.882841) (width 0.3) (layer "B.Cu") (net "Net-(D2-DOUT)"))
 (segment (start 175.26 121.92) (end 175.26 117.26) (width 0.3) (layer "F.Cu") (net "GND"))
 (segment (start 160 116.2) (end 165.9 116.2) (width 0.3) (layer "F.Cu") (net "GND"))
 (segment (start 128.6 97.29) (end 128.6 116.5) (width 0.3) (layer "F.Cu") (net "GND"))
 (segment (start 156.43 121.7) (end 156.21 121.92) (width 0.3) (layer "F.Cu") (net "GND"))
 (segment (start 175.26 117.26) (end 174.5 116.5) (width 0.3) (layer "F.Cu") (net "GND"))
 (segment (start 137.16 121.92) (end 137.16 117.26) (width 0.3) (layer "F.Cu") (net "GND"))
 (segment (start 174.5 116.5) (end 171.1 116.5) (width 0.3) (layer "F.Cu") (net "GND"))
 (segment (start 137.16 117.26) (end 136.2 116.3) (width 0.3) (layer "F.Cu") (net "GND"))
 (segment (start 159.1 121.7) (end 156.43 121.7) (width 0.3) (layer "F.Cu") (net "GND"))
 (segment (start 124.55 93.24) (end 128.6 97.29) (width 0.3) (layer "F.Cu") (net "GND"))
 (segment (start 165.9 116.2) (end 166.2 115.9) (width 0.3) (layer "F.Cu") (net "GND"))
 (segment (start 171.1 116.5) (end 170.7 116.1) (width 0.3) (layer "F.Cu") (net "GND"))
 (via (at 136.2 116.3) (size 0.6) (drill 0.3) (layers "F.Cu" "B.Cu") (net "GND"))
 (via (at 128.6 116.5) (size 0.6) (drill 0.3) (layers "F.Cu" "B.Cu") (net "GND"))
 (via (at 160 116.2) (size 0.6) (drill 0.3) (layers "F.Cu" "B.Cu") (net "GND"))
 (via (at 159.1 121.7) (size 0.6) (drill 0.3) (layers "F.Cu" "B.Cu") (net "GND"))
 (via (at 166.2 115.9) (size 0.6) (drill 0.3) (layers "F.Cu" "B.Cu") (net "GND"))
 (via (at 170.7 116.1) (size 0.6) (drill 0.3) (layers "F.Cu" "B.Cu") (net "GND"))
 (segment (start 128.6 116.5) (end 128.6 116.582843) (width 0.3) (layer "B.Cu") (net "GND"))
 (segment (start 149.799999 117.800001) (end 151.8 115.8) (width 0.3) (layer "B.Cu") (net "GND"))
 (segment (start 179.8 102.542943) (end 179.8 104.38) (width 0.3) (layer "B.Cu") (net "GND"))
 (segment (start 179.8 104.38) (end 178.6 105.58) (width 0.3) (layer "B.Cu") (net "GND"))
 (segment (start 131.9 116.3) (end 130.749999 117.450001) (width 0.3) (layer "B.Cu") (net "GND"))
 (segment (start 149.799999 118.732842) (end 149.197157 118.13) (width 0.3) (layer "B.Cu") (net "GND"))
 (segment (start 160 118.5) (end 160 116.2) (width 0.3) (layer "B.Cu") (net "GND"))
 (segment (start 130.749999 117.450001) (end 130.749999 118.732842) (width 0.3) (layer "B.Cu") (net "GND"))
 (segment (start 170.7 116.1) (end 168.849999 117.950001) (width 0.3) (layer "B.Cu") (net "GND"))
 (segment (start 159.1 119.4) (end 159.1 121.7) (width 0.3) (layer "B.Cu") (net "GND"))
 (segment (start 166.2 116.082843) (end 168.849999 118.732842) (width 0.3) (layer "B.Cu") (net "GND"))
 (segment (start 155.667767 115.8) (end 159.1 119.232233) (width 0.3) (layer "B.Cu") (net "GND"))
 (segment (start 128.6 116.582843) (end 130.749999 118.732842) (width 0.3) (layer "B.Cu") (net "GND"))
 (segment (start 136.2 116.3) (end 131.9 116.3) (width 0.3) (layer "B.Cu") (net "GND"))
 (segment (start 168.849999 118.732842) (end 168.849999 111.092944) (width 0.3) (layer "B.Cu") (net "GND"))
 (segment (start 159.1 119.232233) (end 159.1 119.4) (width 0.3) (layer "B.Cu") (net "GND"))
 (segment (start 151.8 115.8) (end 155.667767 115.8) (width 0.3) (layer "B.Cu") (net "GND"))
 (segment (start 179.097057 101.84) (end 179.8 102.542943) (width 0.3) (layer "B.Cu") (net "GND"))
 (segment (start 149.197157 118.13) (end 142.505634 118.13) (width 0.3) (layer "B.Cu") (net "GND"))
 (segment (start 168.849999 117.950001) (end 168.849999 118.732842) (width 0.3) (layer "B.Cu") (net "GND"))
 (segment (start 149.799999 118.732842) (end 149.799999 117.800001) (width 0.3) (layer "B.Cu") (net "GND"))
 (segment (start 142.505634 118.13) (end 138.715634 121.92) (width 0.3) (layer "B.Cu") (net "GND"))
 (segment (start 178.102943 101.84) (end 179.097057 101.84) (width 0.3) (layer "B.Cu") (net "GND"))
 (segment (start 168.849999 111.092944) (end 178.102943 101.84) (width 0.3) (layer "B.Cu") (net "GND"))
 (segment (start 138.715634 121.92) (end 137.16 121.92) (width 0.3) (layer "B.Cu") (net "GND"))
 (segment (start 159.1 119.4) (end 160 118.5) (width 0.3) (layer "B.Cu") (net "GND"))
 (segment (start 166.2 115.9) (end 166.2 116.082843) (width 0.3) (layer "B.Cu") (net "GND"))
 (segment (start 143.6 120.6) (end 145.2 122.2) (width 0.3) (layer "F.Cu") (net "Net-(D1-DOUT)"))
 (segment (start 143.6 117.1) (end 143.6 120.6) (width 0.3) (layer "F.Cu") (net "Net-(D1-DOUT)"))
 (via (at 145.2 122.2) (size 0.6) (drill 0.3) (layers "F.Cu" "B.Cu") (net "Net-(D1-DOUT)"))
 (via (at 143.6 117.1) (size 0.6) (drill 0.3) (layers "F.Cu" "B.Cu") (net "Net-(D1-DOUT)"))
 (segment (start 137.582841 117.1) (end 143.6 117.1) (width 0.3) (layer "B.Cu") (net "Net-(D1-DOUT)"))
 (segment (start 135.949999 118.732842) (end 137.582841 117.1) (width 0.3) (layer "B.Cu") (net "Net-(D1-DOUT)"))
 (segment (start 147.832841 122.2) (end 149.799999 120.232842) (width 0.3) (layer "B.Cu") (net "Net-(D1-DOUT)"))
 (segment (start 145.2 122.2) (end 147.832841 122.2) (width 0.3) (layer "B.Cu") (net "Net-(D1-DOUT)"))
 (segment (start 139.8 90.7) (end 129.52 100.98) (width 0.3) (layer "F.Cu") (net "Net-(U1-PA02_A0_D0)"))
 (segment (start 129.52 100.98) (end 129.52 123.17) (width 0.3) (layer "F.Cu") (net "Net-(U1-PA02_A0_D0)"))
 (segment (start 129.52 123.17) (end 130.81 124.46) (width 0.3) (layer "F.Cu") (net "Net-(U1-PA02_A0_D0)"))
 (segment (start 139.8 103.4) (end 175.7 103.4) (width 0.3) (layer "F.Cu") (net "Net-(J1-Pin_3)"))
 (segment (start 175.7 103.4) (end 178.8 100.3) (width 0.3) (layer "F.Cu") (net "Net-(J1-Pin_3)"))
 (segment (start 178.8 100.3) (end 180.2 100.3) (width 0.3) (layer "F.Cu") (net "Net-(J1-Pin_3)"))
 (segment (start 139.8 100.86) (end 175.7 100.86) (width 0.3) (layer "F.Cu") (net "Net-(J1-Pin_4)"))
 (segment (start 175.7 100.86) (end 178.8 97.76) (width 0.3) (layer "F.Cu") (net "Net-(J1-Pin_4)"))
 (segment (start 178.8 97.76) (end 180.2 97.76) (width 0.3) (layer "F.Cu") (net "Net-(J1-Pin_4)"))
 (segment (start 130.749999 120.232842) (end 129.855075 120.232842) (width 0.3) (layer "B.Cu") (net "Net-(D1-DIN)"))
 (segment (start 127.95 116.769239) (end 127.95 110.17) (width 0.3) (layer "B.Cu") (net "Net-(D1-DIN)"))
 (segment (start 129.52 119.897767) (end 129.52 118.339239) (width 0.3) (layer "B.Cu") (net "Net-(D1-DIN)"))
 (segment (start 127.95 110.17) (end 139.8 98.32) (width 0.3) (layer "B.Cu") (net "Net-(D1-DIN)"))
 (segment (start 129.52 118.339239) (end 127.95 116.769239) (width 0.3) (layer "B.Cu") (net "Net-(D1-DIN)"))
 (segment (start 129.855075 120.232842) (end 129.52 119.897767) (width 0.3) (layer "B.Cu") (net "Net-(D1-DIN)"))
 (segment (start 144.9 99.7) (end 144.9 99.8) (width 0.3) (layer "F.Cu") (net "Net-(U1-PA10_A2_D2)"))
 (segment (start 139.8 95.78) (end 140.98 95.78) (width 0.3) (layer "F.Cu") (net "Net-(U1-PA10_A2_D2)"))
 (segment (start 140.98 95.78) (end 144.9 99.7) (width 0.3) (layer "F.Cu") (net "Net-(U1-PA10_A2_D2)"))
 (via (at 144.9 99.8) (size 0.6) (drill 0.3) (layers "F.Cu" "B.Cu") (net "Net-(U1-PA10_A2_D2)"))
 (segment (start 144.9 99.8) (end 166.7 121.6) (width 0.3) (layer "B.Cu") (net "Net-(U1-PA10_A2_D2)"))
 (segment (start 166.7 121.6) (end 166.7 122.25) (width 0.3) (layer "B.Cu") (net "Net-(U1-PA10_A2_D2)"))
 (segment (start 166.7 122.25) (end 168.91 124.46) (width 0.3) (layer "B.Cu") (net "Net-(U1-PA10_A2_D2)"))
 (segment (start 149.86 124.46) (end 149.86 117.647056) (width 0.3) (layer "F.Cu") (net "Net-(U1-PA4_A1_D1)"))
 (segment (start 138.65 94.39) (end 139.8 93.24) (width 0.3) (layer "F.Cu") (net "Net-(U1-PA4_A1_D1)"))
 (segment (start 149.86 117.647056) (end 138.65 106.437056) (width 0.3) (layer "F.Cu") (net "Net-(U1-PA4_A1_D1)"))
 (segment (start 138.65 106.437056) (end 138.65 94.39) (width 0.3) (layer "F.Cu") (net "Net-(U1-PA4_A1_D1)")))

